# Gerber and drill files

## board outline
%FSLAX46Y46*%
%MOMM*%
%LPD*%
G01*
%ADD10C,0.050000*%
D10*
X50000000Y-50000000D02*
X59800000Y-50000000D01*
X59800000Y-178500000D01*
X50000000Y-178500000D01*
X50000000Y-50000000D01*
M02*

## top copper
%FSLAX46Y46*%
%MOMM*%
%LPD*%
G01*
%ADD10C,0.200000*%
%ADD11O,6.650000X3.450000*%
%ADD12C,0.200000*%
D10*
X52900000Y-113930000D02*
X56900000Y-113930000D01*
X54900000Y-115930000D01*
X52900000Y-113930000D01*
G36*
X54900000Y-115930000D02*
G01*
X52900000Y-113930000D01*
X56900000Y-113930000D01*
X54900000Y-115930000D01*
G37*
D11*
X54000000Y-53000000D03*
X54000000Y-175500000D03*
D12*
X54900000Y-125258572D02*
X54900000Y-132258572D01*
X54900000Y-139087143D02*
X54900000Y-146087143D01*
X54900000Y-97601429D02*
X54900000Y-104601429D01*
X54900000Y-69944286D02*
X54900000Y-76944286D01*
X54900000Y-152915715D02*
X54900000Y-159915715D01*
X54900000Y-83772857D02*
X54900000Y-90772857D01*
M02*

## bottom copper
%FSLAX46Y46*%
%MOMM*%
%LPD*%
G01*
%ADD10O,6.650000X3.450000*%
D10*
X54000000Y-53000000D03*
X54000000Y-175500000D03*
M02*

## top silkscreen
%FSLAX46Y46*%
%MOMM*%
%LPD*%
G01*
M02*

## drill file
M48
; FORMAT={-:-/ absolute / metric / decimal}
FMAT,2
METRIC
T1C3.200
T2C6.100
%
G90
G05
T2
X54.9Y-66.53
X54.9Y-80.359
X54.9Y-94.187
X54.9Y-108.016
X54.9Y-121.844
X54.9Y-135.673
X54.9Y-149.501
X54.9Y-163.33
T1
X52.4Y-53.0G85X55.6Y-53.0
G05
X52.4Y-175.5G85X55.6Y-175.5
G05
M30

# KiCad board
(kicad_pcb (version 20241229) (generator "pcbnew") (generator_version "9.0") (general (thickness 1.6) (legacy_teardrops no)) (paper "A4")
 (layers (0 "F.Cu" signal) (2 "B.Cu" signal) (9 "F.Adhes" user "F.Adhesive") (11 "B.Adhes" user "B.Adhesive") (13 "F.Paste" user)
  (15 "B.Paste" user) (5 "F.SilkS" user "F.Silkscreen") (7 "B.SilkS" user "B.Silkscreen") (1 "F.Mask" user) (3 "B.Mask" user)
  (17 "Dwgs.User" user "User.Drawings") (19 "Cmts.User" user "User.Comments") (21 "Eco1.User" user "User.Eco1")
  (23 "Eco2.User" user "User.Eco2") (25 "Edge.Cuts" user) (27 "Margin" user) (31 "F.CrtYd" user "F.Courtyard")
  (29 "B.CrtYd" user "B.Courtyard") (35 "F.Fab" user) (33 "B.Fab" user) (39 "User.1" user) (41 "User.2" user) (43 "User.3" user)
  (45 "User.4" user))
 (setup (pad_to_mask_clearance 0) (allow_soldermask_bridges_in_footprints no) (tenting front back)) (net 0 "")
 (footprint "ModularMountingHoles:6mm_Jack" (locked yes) (layer "F.Cu") (at 54.9 94.187143)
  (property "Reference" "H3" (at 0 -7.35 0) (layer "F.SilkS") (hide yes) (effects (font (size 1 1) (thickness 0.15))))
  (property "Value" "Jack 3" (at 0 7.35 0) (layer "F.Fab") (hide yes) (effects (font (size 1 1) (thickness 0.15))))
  (pad "" np_thru_hole circle (at 0 0) (size 6.1 6.1) (drill 6.1) (layers "*.Cu" "*.Mask")))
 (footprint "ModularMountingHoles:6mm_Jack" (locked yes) (layer "F.Cu") (at 54.9 163.33)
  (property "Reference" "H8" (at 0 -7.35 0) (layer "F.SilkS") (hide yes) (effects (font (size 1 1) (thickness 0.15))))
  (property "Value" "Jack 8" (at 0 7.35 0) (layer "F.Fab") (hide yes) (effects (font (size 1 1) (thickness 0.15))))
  (pad "" np_thru_hole circle (at 0 0) (size 6.1 6.1) (drill 6.1) (layers "*.Cu" "*.Mask")))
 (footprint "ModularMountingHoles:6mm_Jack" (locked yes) (layer "F.Cu") (at 54.9 149.501429)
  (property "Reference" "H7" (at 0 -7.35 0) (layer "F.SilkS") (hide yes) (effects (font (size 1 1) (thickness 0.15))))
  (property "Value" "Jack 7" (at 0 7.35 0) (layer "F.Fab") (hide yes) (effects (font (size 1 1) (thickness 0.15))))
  (pad "" np_thru_hole circle (at 0 0) (size 6.1 6.1) (drill 6.1) (layers "*.Cu" "*.Mask")))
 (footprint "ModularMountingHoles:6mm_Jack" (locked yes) (layer "F.Cu") (at 54.9 121.844286)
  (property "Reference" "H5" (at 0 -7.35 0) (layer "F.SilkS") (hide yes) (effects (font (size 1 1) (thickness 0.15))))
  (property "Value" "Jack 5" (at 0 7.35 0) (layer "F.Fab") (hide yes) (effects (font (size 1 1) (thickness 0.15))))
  (pad "" np_thru_hole circle (at 0 0) (size 6.1 6.1) (drill 6.1) (layers "*.Cu" "*.Mask")))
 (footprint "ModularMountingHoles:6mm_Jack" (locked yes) (layer "F.Cu") (at 54.9 108.015714)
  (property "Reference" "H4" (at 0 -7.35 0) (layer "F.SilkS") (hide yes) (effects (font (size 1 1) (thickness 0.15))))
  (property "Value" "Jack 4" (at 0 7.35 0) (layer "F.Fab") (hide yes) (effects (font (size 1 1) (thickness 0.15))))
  (pad "" np_thru_hole circle (at 0 0) (size 6.1 6.1) (drill 6.1) (layers "*.Cu" "*.Mask")))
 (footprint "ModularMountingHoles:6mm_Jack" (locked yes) (layer "F.Cu") (at 54.9 135.672857)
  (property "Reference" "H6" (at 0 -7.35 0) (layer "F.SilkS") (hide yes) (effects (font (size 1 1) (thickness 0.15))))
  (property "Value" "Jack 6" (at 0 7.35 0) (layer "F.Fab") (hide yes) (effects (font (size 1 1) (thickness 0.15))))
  (pad "" np_thru_hole circle (at 0 0) (size 6.1 6.1) (drill 6.1) (layers "*.Cu" "*.Mask")))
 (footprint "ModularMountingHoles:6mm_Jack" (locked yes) (layer "F.Cu") (at 54.9 66.53)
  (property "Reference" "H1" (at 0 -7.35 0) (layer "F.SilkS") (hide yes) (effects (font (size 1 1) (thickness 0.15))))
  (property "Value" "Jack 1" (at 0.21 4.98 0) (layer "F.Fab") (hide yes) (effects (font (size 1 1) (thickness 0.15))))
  (pad "" np_thru_hole circle (at 0 0) (size 6.1 6.1) (drill 6.1) (layers "*.Cu" "*.Mask")))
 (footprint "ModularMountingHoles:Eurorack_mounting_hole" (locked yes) (layer "F.Cu") (at 54 53)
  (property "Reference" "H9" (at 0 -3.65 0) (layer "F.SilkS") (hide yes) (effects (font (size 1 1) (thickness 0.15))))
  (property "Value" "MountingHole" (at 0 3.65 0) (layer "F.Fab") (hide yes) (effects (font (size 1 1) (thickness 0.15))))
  (pad "1" thru_hole oval (at 0 0) (size 6.65 3.45) (drill oval 6.4 3.2) (layers "*.Cu" "*.Mask") (remove_unused_layers no) (zone_connect 2)))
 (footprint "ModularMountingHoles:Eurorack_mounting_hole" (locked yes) (layer "F.Cu") (at 54 175.5)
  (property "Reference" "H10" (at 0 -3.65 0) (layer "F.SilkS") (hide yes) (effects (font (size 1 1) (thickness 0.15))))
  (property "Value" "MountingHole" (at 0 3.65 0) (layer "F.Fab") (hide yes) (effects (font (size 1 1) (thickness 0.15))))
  (pad "1" thru_hole oval (at 0 0) (size 6.65 3.45) (drill oval 6.4 3.2) (layers "*.Cu" "*.Mask") (remove_unused_layers no) (zone_connect 2)))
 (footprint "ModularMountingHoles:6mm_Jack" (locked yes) (layer "F.Cu") (at 54.9 80.358571)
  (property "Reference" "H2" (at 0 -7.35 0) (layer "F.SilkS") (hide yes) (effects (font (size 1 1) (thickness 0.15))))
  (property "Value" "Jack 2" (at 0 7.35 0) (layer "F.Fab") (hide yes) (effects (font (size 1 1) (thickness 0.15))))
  (pad "" np_thru_hole circle (at 0 0) (size 6.1 6.1) (drill 6.1) (layers "*.Cu" "*.Mask")))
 (gr_poly (pts (xy 52.9 113.93) (xy 56.9 113.93) (xy 54.9 115.93)) (stroke (width 0.2) (type solid)) (fill yes) (layer "F.Cu"))
 (gr_rect (start 50 50) (end 59.8 178.5) (stroke (width 0.05) (type solid)) (fill no) (locked yes) (layer "Edge.Cuts"))
 (segment (start 54.9 125.258572) (end 54.9 132.258572) (width 0.2) (locked yes) (layer "F.Cu") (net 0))
 (segment (start 54.9 139.087143) (end 54.9 146.087143) (width 0.2) (locked yes) (layer "F.Cu") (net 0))
 (segment (start 54.9 97.601429) (end 54.9 104.601429) (width 0.2) (locked yes) (layer "F.Cu") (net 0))
 (segment (start 54.9 69.944286) (end 54.9 76.944286) (width 0.2) (locked yes) (layer "F.Cu") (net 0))
 (segment (start 54.9 152.915715) (end 54.9 159.915715) (width 0.2) (locked yes) (layer "F.Cu") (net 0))
 (segment (start 54.9 83.772857) (end 54.9 90.772857) (width 0.2) (locked yes) (layer "F.Cu") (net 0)))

